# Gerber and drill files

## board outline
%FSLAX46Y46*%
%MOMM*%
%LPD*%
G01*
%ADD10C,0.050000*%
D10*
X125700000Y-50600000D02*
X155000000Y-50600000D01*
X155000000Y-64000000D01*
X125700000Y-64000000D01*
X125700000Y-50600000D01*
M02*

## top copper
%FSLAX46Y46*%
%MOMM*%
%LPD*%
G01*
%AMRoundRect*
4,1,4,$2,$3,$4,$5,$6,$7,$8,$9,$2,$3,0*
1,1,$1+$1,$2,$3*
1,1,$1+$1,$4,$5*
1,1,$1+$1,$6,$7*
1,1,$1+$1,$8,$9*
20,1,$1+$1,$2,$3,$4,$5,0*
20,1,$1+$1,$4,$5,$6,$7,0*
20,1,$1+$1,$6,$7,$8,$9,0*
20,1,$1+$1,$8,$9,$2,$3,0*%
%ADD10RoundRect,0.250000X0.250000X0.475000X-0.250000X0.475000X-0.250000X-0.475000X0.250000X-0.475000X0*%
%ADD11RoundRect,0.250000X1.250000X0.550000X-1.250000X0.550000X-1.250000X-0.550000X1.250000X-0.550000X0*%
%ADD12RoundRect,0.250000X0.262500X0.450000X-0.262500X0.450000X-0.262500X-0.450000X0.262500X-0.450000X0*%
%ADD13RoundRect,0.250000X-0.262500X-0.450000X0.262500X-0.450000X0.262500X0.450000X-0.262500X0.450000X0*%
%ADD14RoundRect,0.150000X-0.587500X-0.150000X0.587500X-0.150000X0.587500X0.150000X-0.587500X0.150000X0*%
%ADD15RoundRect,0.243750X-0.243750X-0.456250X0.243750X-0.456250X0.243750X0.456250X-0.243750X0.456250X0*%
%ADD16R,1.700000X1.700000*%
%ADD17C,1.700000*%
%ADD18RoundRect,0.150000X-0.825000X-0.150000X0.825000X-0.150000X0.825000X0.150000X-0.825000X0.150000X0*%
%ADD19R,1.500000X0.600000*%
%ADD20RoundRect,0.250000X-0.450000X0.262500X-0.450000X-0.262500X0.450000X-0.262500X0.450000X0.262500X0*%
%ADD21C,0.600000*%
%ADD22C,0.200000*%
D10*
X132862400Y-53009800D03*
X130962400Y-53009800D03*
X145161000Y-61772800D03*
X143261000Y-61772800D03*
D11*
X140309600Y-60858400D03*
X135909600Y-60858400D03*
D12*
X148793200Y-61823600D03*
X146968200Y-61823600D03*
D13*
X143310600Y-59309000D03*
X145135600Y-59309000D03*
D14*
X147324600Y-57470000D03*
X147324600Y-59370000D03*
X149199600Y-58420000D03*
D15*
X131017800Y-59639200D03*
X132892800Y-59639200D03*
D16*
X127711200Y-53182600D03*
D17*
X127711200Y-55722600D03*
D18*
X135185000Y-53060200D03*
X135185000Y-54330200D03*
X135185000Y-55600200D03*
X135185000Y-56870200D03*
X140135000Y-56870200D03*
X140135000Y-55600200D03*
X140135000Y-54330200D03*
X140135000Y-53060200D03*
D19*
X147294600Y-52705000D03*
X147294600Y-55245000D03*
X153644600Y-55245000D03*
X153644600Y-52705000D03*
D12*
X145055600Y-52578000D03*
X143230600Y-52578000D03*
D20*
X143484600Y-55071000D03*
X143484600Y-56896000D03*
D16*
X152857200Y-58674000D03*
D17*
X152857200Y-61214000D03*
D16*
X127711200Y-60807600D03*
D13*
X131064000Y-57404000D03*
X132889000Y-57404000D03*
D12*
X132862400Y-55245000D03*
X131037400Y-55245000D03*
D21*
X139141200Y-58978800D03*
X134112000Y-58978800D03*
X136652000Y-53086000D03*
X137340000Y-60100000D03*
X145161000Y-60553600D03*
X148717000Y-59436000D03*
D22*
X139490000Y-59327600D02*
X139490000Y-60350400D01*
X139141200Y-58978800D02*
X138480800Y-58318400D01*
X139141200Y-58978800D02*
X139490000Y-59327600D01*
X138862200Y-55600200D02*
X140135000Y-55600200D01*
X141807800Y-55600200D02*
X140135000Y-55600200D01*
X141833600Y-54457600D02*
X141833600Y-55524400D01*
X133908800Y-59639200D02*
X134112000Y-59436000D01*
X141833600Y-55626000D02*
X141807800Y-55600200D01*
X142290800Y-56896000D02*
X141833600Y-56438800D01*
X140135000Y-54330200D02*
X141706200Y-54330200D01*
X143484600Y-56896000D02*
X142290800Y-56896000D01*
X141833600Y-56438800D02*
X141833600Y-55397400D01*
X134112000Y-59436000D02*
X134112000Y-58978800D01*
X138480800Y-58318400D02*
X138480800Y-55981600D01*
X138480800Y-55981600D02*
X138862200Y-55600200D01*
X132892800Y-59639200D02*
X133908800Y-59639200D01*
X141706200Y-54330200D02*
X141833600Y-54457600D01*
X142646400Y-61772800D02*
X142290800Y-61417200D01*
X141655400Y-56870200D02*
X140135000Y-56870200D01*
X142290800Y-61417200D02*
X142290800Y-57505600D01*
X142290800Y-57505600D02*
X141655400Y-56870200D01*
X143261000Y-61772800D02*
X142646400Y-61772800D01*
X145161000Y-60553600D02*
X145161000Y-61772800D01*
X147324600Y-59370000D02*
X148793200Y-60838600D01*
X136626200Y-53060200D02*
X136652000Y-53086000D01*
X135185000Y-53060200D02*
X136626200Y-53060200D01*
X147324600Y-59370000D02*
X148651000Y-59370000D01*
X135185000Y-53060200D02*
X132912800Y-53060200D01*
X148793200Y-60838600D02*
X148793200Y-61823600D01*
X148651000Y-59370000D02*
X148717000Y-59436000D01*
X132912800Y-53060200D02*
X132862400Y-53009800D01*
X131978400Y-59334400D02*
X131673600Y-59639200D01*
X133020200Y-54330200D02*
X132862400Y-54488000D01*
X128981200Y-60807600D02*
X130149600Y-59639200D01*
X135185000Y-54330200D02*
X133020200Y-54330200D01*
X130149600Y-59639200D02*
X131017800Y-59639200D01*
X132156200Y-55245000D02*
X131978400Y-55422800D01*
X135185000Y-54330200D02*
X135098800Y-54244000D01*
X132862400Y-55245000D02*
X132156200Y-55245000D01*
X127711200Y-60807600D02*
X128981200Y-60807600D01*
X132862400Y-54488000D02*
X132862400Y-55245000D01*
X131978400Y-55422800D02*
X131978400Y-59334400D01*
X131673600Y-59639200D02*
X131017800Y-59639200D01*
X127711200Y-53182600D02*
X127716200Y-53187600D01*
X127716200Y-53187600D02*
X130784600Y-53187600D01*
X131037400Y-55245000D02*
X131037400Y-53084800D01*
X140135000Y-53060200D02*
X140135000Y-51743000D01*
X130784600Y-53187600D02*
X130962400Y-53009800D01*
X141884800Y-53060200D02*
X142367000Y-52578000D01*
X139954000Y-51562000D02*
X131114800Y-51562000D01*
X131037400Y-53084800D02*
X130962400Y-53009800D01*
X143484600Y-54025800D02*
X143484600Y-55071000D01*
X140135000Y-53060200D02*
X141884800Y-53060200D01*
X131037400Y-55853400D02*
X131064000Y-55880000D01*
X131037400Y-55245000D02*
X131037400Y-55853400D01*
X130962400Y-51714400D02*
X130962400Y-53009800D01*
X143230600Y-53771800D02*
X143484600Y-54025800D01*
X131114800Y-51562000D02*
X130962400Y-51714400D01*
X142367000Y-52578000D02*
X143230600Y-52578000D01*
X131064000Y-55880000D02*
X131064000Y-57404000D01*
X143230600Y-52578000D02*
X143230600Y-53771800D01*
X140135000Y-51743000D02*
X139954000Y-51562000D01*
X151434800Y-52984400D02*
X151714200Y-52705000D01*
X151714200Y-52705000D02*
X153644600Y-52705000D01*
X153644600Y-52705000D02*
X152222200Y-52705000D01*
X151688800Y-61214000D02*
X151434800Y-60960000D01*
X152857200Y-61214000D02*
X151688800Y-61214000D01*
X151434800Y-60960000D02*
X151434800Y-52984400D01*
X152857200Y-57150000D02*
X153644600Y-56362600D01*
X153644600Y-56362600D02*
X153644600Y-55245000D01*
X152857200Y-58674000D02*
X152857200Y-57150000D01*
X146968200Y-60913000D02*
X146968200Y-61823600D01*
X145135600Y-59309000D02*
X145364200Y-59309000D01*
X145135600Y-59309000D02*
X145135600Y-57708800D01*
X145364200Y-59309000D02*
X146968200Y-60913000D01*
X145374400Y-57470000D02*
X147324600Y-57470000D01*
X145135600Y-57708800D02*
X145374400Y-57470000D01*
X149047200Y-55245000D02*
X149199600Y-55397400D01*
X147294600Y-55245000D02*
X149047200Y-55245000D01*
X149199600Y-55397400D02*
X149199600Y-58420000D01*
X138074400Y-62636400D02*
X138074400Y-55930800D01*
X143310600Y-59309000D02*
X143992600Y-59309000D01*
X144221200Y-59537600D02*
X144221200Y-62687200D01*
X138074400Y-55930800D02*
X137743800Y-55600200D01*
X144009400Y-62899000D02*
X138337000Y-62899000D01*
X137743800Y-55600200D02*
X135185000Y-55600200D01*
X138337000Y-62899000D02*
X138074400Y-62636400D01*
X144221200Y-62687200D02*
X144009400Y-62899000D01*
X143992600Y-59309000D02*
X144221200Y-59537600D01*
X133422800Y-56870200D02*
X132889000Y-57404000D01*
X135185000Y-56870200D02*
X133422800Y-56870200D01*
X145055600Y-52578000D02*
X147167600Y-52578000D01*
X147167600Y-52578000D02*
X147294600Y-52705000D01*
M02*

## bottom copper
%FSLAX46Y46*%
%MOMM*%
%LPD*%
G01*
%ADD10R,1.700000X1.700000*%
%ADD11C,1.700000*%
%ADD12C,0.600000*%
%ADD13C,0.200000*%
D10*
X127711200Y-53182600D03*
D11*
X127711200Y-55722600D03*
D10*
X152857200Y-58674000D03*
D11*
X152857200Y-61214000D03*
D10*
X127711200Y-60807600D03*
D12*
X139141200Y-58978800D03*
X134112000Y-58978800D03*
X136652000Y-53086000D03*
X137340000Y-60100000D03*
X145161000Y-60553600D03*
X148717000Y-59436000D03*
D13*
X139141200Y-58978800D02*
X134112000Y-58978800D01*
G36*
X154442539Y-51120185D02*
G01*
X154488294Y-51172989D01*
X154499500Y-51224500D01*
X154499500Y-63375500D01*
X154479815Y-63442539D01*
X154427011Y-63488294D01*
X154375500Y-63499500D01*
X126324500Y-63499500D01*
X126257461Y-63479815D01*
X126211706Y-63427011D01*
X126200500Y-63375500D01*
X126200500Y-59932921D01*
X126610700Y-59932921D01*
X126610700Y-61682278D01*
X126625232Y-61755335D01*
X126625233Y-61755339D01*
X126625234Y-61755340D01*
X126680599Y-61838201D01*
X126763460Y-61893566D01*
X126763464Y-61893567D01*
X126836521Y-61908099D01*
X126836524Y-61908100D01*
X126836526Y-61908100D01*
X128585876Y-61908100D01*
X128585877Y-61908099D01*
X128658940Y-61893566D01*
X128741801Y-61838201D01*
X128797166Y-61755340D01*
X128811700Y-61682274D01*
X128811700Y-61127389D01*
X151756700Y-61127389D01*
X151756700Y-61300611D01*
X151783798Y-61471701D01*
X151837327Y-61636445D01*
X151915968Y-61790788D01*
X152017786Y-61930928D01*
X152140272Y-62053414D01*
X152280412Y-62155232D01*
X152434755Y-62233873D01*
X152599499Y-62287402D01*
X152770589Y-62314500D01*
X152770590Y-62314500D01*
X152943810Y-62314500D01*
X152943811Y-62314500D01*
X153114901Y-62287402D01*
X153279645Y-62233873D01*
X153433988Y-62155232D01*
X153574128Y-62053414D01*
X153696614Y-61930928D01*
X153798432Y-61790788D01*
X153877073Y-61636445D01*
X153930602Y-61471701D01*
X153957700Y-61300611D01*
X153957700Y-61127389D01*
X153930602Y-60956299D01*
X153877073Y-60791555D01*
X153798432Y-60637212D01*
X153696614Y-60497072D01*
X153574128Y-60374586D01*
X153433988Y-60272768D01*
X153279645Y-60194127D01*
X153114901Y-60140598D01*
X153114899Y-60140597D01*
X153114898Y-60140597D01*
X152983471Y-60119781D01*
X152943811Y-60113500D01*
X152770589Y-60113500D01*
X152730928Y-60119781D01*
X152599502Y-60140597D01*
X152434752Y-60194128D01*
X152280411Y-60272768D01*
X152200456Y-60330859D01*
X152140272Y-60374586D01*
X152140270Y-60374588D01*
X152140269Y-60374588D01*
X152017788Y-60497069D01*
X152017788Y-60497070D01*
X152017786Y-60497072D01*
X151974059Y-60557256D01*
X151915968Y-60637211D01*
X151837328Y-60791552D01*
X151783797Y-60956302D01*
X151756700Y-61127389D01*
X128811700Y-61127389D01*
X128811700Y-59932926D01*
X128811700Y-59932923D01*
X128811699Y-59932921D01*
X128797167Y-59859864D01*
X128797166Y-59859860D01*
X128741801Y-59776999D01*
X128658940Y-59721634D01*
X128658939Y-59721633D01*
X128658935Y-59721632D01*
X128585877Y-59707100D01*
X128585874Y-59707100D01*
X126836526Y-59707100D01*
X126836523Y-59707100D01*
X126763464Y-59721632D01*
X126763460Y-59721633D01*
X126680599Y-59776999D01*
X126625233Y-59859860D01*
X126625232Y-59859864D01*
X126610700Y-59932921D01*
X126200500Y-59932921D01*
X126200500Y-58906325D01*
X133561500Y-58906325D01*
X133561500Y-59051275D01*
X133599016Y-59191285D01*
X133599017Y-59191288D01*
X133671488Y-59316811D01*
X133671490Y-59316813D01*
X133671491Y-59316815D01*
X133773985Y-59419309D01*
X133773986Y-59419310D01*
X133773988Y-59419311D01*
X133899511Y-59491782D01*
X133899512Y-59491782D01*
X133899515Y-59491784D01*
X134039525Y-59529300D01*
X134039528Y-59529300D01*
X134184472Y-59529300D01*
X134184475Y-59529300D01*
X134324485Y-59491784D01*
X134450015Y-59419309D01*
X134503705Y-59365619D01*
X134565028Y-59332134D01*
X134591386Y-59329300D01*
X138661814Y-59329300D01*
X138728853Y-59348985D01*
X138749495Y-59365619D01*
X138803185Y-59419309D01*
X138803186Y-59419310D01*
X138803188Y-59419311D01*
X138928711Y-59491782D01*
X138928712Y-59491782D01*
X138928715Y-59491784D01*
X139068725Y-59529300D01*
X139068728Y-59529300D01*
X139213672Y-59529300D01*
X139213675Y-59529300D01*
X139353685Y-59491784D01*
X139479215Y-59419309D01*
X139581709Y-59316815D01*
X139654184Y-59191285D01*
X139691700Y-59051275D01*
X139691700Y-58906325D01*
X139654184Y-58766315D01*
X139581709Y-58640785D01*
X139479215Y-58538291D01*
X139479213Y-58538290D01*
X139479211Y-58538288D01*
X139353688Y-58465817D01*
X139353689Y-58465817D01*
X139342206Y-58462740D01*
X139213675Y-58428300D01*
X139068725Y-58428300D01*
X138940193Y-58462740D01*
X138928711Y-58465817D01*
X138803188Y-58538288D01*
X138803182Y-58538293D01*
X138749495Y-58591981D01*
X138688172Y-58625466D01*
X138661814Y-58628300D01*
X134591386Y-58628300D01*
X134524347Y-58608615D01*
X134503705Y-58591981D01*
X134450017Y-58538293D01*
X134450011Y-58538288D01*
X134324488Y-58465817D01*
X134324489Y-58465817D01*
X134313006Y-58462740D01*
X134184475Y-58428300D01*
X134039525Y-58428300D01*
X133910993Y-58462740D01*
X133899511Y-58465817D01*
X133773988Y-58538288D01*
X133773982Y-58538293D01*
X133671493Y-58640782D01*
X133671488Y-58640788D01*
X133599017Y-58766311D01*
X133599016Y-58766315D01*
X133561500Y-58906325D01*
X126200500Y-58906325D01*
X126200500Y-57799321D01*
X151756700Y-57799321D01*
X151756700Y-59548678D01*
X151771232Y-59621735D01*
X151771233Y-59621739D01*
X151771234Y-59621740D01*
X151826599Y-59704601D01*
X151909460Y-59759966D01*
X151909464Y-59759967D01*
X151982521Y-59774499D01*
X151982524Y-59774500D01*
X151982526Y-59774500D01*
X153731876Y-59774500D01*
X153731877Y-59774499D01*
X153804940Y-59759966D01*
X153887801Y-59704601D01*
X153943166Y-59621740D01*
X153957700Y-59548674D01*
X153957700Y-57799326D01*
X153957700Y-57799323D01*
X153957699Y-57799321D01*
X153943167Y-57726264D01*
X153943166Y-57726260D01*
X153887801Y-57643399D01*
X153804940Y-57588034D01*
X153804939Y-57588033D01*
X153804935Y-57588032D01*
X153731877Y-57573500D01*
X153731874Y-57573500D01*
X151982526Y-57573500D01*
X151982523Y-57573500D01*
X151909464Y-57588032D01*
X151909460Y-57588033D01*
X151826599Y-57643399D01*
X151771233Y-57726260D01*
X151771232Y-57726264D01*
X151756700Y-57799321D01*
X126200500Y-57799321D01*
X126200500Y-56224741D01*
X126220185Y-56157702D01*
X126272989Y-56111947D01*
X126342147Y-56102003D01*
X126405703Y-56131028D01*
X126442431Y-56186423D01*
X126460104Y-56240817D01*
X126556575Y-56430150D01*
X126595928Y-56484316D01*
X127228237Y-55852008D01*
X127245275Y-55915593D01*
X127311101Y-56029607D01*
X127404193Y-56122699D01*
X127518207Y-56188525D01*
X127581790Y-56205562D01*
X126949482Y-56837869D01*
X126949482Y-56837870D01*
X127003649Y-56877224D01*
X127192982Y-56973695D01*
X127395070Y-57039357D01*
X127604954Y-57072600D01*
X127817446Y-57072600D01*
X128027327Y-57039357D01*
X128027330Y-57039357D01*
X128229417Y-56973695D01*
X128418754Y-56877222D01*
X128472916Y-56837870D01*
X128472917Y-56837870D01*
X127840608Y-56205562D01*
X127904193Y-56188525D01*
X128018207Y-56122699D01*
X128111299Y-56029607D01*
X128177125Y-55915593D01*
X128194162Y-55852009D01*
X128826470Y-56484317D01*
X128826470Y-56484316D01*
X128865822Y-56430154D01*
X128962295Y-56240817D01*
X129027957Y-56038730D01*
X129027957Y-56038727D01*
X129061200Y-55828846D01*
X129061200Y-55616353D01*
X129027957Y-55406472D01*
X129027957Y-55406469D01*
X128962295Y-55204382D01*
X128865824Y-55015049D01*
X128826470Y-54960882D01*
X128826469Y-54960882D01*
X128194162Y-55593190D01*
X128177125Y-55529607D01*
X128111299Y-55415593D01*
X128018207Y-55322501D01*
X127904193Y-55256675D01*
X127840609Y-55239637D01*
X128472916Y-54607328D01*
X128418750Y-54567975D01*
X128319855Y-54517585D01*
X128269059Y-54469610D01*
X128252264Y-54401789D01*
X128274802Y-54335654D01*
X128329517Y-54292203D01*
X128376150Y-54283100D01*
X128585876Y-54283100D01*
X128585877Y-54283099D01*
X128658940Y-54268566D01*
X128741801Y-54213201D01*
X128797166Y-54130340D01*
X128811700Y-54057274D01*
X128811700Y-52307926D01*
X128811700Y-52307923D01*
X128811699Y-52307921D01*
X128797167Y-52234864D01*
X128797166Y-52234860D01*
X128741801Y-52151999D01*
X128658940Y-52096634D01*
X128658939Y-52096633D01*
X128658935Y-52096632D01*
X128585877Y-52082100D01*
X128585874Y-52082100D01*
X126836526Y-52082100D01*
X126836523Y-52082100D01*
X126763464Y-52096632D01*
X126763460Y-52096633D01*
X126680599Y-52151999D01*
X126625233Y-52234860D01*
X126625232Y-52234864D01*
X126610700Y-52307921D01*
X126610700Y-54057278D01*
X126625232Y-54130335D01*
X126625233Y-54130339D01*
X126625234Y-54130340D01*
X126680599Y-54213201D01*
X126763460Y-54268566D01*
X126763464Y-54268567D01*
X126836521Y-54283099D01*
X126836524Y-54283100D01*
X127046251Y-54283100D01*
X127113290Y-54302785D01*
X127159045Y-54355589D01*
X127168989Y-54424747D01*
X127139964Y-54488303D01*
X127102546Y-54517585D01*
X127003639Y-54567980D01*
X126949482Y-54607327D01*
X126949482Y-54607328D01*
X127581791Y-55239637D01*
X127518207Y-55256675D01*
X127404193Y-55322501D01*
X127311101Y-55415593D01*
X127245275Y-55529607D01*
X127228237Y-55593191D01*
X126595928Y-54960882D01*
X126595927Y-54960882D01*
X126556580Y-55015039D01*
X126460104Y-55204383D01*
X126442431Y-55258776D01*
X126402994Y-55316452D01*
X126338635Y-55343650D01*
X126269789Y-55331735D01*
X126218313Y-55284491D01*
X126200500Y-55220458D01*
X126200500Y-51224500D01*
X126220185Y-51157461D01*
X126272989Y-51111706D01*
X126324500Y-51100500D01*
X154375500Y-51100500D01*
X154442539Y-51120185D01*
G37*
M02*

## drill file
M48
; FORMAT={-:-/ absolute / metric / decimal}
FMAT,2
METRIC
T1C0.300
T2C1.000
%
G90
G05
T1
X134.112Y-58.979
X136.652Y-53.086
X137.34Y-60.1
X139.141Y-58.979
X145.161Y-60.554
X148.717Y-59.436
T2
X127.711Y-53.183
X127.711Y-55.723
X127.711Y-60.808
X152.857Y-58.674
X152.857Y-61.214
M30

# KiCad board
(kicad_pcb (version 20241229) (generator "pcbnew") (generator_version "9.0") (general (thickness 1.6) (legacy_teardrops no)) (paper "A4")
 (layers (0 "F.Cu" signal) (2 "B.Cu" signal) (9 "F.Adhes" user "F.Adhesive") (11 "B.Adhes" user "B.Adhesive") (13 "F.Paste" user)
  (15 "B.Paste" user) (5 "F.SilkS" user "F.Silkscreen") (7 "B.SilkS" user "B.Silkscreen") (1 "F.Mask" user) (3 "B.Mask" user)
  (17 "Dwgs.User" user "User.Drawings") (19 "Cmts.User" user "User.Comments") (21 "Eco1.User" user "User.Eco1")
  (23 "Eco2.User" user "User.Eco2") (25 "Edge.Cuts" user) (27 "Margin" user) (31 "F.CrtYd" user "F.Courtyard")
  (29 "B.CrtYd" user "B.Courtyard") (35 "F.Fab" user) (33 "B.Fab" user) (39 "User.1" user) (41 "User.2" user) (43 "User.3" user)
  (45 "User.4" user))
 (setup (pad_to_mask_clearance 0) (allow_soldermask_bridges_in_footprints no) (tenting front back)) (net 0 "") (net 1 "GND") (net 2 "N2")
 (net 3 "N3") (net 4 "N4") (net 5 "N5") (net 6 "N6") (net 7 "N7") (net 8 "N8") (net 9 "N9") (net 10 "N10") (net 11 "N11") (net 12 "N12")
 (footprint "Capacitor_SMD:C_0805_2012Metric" (layer "F.Cu") (at 131.9124 53.0098 180)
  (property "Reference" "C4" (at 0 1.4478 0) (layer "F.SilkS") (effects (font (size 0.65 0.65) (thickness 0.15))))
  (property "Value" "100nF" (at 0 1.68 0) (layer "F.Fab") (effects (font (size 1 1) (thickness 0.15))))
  (pad "1" smd roundrect (at -0.95 0 180) (size 1 1.45) (layers "F.Cu" "F.Mask" "F.Paste") (roundrect_rratio 0.25) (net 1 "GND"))
  (pad "2" smd roundrect (at 0.95 0 180) (size 1 1.45) (layers "F.Cu" "F.Mask" "F.Paste") (roundrect_rratio 0.25) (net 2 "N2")))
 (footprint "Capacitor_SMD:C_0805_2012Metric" (layer "F.Cu") (at 144.211 61.7728 180)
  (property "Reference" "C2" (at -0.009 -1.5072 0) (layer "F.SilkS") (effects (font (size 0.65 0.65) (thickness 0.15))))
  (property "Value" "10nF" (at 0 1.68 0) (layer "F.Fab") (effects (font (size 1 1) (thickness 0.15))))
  (pad "1" smd roundrect (at -0.95 0 180) (size 1 1.45) (layers "F.Cu" "F.Mask" "F.Paste") (roundrect_rratio 0.25) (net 1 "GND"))
  (pad "2" smd roundrect (at 0.95 0 180) (size 1 1.45) (layers "F.Cu" "F.Mask" "F.Paste") (roundrect_rratio 0.25) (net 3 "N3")))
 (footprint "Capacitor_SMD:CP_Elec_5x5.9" (layer "F.Cu") (at 138.1096 60.8584 180)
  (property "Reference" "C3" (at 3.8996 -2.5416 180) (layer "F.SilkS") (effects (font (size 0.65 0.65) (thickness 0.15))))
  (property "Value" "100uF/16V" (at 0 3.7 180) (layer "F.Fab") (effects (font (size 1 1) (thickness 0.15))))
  (pad "1" smd roundrect (at -2.2 0 180) (size 3 1.6) (layers "F.Cu" "F.Mask" "F.Paste") (roundrect_rratio 0.15625) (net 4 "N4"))
  (pad "2" smd roundrect (at 2.2 0 180) (size 3 1.6) (layers "F.Cu" "F.Mask" "F.Paste") (roundrect_rratio 0.15625) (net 1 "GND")))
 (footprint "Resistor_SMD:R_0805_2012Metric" (layer "F.Cu") (at 147.8807 61.8236 180)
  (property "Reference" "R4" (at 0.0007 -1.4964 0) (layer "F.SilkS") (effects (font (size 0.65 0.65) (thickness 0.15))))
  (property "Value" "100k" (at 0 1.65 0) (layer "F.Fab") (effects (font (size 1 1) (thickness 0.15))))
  (pad "1" smd roundrect (at -0.9125 0 180) (size 1.025 1.4) (layers "F.Cu" "F.Mask" "F.Paste") (roundrect_rratio 0.243902) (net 1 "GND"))
  (pad "2" smd roundrect (at 0.9125 0 180) (size 1.025 1.4) (layers "F.Cu" "F.Mask" "F.Paste") (roundrect_rratio 0.243902) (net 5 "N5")))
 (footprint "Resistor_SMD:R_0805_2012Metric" (layer "F.Cu") (at 144.2231 59.309)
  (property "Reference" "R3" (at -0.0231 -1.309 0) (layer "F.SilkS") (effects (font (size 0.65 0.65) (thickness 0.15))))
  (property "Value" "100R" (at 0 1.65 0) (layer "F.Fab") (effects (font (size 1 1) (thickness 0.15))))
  (pad "1" smd roundrect (at -0.9125 0) (size 1.025 1.4) (layers "F.Cu" "F.Mask" "F.Paste") (roundrect_rratio 0.243902) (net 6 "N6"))
  (pad "2" smd roundrect (at 0.9125 0) (size 1.025 1.4) (layers "F.Cu" "F.Mask" "F.Paste") (roundrect_rratio 0.243902) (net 5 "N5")))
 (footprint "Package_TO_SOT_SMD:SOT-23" (layer "F.Cu") (at 148.2621 58.42)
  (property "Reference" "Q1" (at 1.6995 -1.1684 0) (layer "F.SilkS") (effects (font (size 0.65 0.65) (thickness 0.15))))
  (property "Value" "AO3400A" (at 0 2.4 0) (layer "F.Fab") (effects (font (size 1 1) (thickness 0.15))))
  (pad "1" smd roundrect (at -0.9375 -0.95) (size 1.475 0.6) (layers "F.Cu" "F.Mask" "F.Paste") (roundrect_rratio 0.25) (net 5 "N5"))
  (pad "2" smd roundrect (at -0.9375 0.95) (size 1.475 0.6) (layers "F.Cu" "F.Mask" "F.Paste") (roundrect_rratio 0.25) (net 1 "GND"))
  (pad "3" smd roundrect (at 0.9375 0) (size 1.475 0.6) (layers "F.Cu" "F.Mask" "F.Paste") (roundrect_rratio 0.25) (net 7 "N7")))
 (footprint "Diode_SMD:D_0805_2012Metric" (layer "F.Cu") (at 131.9553 59.6392)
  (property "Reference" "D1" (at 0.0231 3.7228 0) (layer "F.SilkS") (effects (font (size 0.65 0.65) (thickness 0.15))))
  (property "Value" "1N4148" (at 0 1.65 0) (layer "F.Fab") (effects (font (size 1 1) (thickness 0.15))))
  (pad "1" smd roundrect (at -0.9375 0) (size 0.975 1.4) (layers "F.Cu" "F.Mask" "F.Paste") (roundrect_rratio 0.25) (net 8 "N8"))
  (pad "2" smd roundrect (at 0.9375 0) (size 0.975 1.4) (layers "F.Cu" "F.Mask" "F.Paste") (roundrect_rratio 0.25) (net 4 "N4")))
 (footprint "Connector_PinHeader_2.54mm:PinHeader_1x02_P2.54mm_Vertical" (layer "F.Cu") (at 127.7112 53.1826)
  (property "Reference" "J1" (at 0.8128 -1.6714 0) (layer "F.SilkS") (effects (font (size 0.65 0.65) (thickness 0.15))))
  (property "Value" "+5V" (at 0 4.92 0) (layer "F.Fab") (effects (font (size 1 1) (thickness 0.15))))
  (pad "1" thru_hole rect (at 0 0) (size 1.7 1.7) (drill 1) (layers "*.Cu" "*.Mask") (remove_unused_layers no) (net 2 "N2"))
  (pad "2" thru_hole circle (at 0 2.54) (size 1.7 1.7) (drill 1) (layers "*.Cu" "*.Mask") (remove_unused_layers no) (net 1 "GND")))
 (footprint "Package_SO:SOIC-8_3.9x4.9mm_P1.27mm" (layer "F.Cu") (at 137.66 54.9652)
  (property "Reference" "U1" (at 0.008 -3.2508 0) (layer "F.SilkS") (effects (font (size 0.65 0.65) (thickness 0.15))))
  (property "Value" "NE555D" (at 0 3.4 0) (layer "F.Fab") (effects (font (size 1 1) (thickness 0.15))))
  (pad "1" smd roundrect (at -2.475 -1.905) (size 1.95 0.6) (layers "F.Cu" "F.Mask" "F.Paste") (roundrect_rratio 0.25) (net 1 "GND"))
  (pad "2" smd roundrect (at -2.475 -0.635) (size 1.95 0.6) (layers "F.Cu" "F.Mask" "F.Paste") (roundrect_rratio 0.25) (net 8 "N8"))
  (pad "3" smd roundrect (at -2.475 0.635) (size 1.95 0.6) (layers "F.Cu" "F.Mask" "F.Paste") (roundrect_rratio 0.25) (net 6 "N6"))
  (pad "4" smd roundrect (at -2.475 1.905) (size 1.95 0.6) (layers "F.Cu" "F.Mask" "F.Paste") (roundrect_rratio 0.25) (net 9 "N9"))
  (pad "5" smd roundrect (at 2.475 1.905) (size 1.95 0.6) (layers "F.Cu" "F.Mask" "F.Paste") (roundrect_rratio 0.25) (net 3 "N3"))
  (pad "6" smd roundrect (at 2.475 0.635) (size 1.95 0.6) (layers "F.Cu" "F.Mask" "F.Paste") (roundrect_rratio 0.25) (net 4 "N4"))
  (pad "7" smd roundrect (at 2.475 -0.635) (size 1.95 0.6) (layers "F.Cu" "F.Mask" "F.Paste") (roundrect_rratio 0.25) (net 4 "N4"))
  (pad "8" smd roundrect (at 2.475 -1.905) (size 1.95 0.6) (layers "F.Cu" "F.Mask" "F.Paste") (roundrect_rratio 0.25) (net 2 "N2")))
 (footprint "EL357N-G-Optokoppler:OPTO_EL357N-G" (layer "F.Cu") (at 150.4696 53.975)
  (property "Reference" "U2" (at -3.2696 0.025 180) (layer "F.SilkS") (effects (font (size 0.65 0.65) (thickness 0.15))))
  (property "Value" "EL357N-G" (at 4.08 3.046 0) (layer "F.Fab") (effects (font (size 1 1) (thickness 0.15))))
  (pad "1" smd rect (at -3.175 -1.27) (size 1.5 0.6) (layers "F.Cu" "F.Mask" "F.Paste") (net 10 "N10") (solder_mask_margin 0.102))
  (pad "2" smd rect (at -3.175 1.27) (size 1.5 0.6) (layers "F.Cu" "F.Mask" "F.Paste") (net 7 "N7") (solder_mask_margin 0.102))
  (pad "3" smd rect (at 3.175 1.27) (size 1.5 0.6) (layers "F.Cu" "F.Mask" "F.Paste") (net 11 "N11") (solder_mask_margin 0.102))
  (pad "4" smd rect (at 3.175 -1.27) (size 1.5 0.6) (layers "F.Cu" "F.Mask" "F.Paste") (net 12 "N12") (solder_mask_margin 0.102)))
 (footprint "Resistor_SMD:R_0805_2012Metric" (layer "F.Cu") (at 144.1431 52.578 180)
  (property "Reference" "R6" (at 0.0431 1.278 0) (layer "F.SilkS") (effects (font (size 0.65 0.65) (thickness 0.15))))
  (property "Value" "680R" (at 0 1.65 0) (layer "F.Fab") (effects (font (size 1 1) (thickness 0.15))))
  (pad "1" smd roundrect (at -0.9125 0 180) (size 1.025 1.4) (layers "F.Cu" "F.Mask" "F.Paste") (roundrect_rratio 0.243902) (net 10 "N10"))
  (pad "2" smd roundrect (at 0.9125 0 180) (size 1.025 1.4) (layers "F.Cu" "F.Mask" "F.Paste") (roundrect_rratio 0.243902) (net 2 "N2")))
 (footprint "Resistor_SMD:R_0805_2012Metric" (layer "F.Cu") (at 143.4846 55.9835 -90)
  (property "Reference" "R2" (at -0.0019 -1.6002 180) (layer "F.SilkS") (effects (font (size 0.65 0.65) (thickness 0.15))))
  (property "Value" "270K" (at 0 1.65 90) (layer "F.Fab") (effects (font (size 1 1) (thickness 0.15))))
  (pad "1" smd roundrect (at -0.9125 0 270) (size 1.025 1.4) (layers "F.Cu" "F.Mask" "F.Paste") (roundrect_rratio 0.243902) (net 2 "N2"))
  (pad "2" smd roundrect (at 0.9125 0 270) (size 1.025 1.4) (layers "F.Cu" "F.Mask" "F.Paste") (roundrect_rratio 0.243902) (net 4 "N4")))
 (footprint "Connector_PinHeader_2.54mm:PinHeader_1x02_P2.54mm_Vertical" (layer "F.Cu") (at 152.8572 58.674)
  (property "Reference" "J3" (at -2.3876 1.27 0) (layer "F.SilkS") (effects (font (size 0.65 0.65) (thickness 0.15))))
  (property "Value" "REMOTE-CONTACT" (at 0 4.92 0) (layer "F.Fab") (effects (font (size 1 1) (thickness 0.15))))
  (pad "1" thru_hole rect (at 0 0) (size 1.7 1.7) (drill 1) (layers "*.Cu" "*.Mask") (remove_unused_layers no) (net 11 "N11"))
  (pad "2" thru_hole circle (at 0 2.54) (size 1.7 1.7) (drill 1) (layers "*.Cu" "*.Mask") (remove_unused_layers no) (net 12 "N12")))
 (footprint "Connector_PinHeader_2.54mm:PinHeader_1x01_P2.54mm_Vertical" (layer "F.Cu") (at 127.7112 60.8076)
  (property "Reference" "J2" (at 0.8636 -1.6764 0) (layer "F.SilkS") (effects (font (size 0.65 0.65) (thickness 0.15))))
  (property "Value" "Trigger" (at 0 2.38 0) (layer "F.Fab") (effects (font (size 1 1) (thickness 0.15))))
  (pad "1" thru_hole rect (at 0 0) (size 1.7 1.7) (drill 1) (layers "*.Cu" "*.Mask") (remove_unused_layers no) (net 8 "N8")))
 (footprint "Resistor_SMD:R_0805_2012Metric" (layer "F.Cu") (at 131.9765 57.404)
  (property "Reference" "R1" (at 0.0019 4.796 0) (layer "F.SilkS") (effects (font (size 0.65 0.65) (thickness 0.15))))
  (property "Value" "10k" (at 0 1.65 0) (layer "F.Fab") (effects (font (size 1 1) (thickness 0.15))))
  (pad "1" smd roundrect (at -0.9125 0) (size 1.025 1.4) (layers "F.Cu" "F.Mask" "F.Paste") (roundrect_rratio 0.243902) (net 2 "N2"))
  (pad "2" smd roundrect (at 0.9125 0) (size 1.025 1.4) (layers "F.Cu" "F.Mask" "F.Paste") (roundrect_rratio 0.243902) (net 9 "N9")))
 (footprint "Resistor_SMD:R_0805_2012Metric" (layer "F.Cu") (at 131.9499 55.245 180)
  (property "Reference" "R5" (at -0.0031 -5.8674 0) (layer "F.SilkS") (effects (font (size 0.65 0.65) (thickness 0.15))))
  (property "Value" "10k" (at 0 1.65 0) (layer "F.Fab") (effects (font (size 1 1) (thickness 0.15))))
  (pad "1" smd roundrect (at -0.9125 0 180) (size 1.025 1.4) (layers "F.Cu" "F.Mask" "F.Paste") (roundrect_rratio 0.243902) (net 8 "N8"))
  (pad "2" smd roundrect (at 0.9125 0 180) (size 1.025 1.4) (layers "F.Cu" "F.Mask" "F.Paste") (roundrect_rratio 0.243902) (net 2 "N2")))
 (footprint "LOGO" (layer "B.Cu") (at 140.84617 57.489081 180)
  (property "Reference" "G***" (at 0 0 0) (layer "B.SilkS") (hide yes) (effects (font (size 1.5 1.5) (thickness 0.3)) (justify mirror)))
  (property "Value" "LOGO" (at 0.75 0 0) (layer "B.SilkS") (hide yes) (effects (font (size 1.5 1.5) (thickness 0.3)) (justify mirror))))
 (gr_rect (start 125.7 50.6) (end 155 64) (stroke (width 0.05) (type default)) (fill no) (layer "Edge.Cuts"))
 (segment (start 139.49 59.3276) (end 139.49 60.3504) (width 0.2) (layer "F.Cu") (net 4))
 (segment (start 139.1412 58.9788) (end 138.4808 58.3184) (width 0.2) (layer "F.Cu") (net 4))
 (segment (start 139.1412 58.9788) (end 139.49 59.3276) (width 0.2) (layer "F.Cu") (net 4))
 (segment (start 138.8622 55.6002) (end 140.135 55.6002) (width 0.2) (layer "F.Cu") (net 4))
 (segment (start 141.8078 55.6002) (end 140.135 55.6002) (width 0.2) (layer "F.Cu") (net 4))
 (segment (start 141.8336 54.4576) (end 141.8336 55.5244) (width 0.2) (layer "F.Cu") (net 4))
 (segment (start 133.9088 59.6392) (end 134.112 59.436) (width 0.2) (layer "F.Cu") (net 4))
 (segment (start 141.8336 55.626) (end 141.8078 55.6002) (width 0.2) (layer "F.Cu") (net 4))
 (segment (start 142.2908 56.896) (end 141.8336 56.4388) (width 0.2) (layer "F.Cu") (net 4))
 (segment (start 140.135 54.3302) (end 141.7062 54.3302) (width 0.2) (layer "F.Cu") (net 4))
 (segment (start 143.4846 56.896) (end 142.2908 56.896) (width 0.2) (layer "F.Cu") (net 4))
 (segment (start 141.8336 56.4388) (end 141.8336 55.3974) (width 0.2) (layer "F.Cu") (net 4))
 (segment (start 134.112 59.436) (end 134.112 58.9788) (width 0.2) (layer "F.Cu") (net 4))
 (segment (start 138.4808 58.3184) (end 138.4808 55.9816) (width 0.2) (layer "F.Cu") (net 4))
 (segment (start 138.4808 55.9816) (end 138.8622 55.6002) (width 0.2) (layer "F.Cu") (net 4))
 (segment (start 132.8928 59.6392) (end 133.9088 59.6392) (width 0.2) (layer "F.Cu") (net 4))
 (segment (start 141.7062 54.3302) (end 141.8336 54.4576) (width 0.2) (layer "F.Cu") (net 4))
 (via (at 139.1412 58.9788) (size 0.6) (drill 0.3) (layers "F.Cu" "B.Cu") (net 4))
 (via (at 134.112 58.9788) (size 0.6) (drill 0.3) (layers "F.Cu" "B.Cu") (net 4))
 (segment (start 139.1412 58.9788) (end 134.112 58.9788) (width 0.2) (layer "B.Cu") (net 4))
 (segment (start 142.6464 61.7728) (end 142.2908 61.4172) (width 0.2) (layer "F.Cu") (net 3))
 (segment (start 141.6554 56.8702) (end 140.135 56.8702) (width 0.2) (layer "F.Cu") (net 3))
 (segment (start 142.2908 61.4172) (end 142.2908 57.5056) (width 0.2) (layer "F.Cu") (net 3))
 (segment (start 142.2908 57.5056) (end 141.6554 56.8702) (width 0.2) (layer "F.Cu") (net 3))
 (segment (start 143.261 61.7728) (end 142.6464 61.7728) (width 0.2) (layer "F.Cu") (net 3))
 (segment (start 145.161 60.5536) (end 145.161 61.7728) (width 0.2) (layer "F.Cu") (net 1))
 (segment (start 147.3246 59.37) (end 148.7932 60.8386) (width 0.2) (layer "F.Cu") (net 1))
 (segment (start 136.6262 53.0602) (end 136.652 53.086) (width 0.2) (layer "F.Cu") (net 1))
 (segment (start 135.185 53.0602) (end 136.6262 53.0602) (width 0.2) (layer "F.Cu") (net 1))
 (segment (start 147.3246 59.37) (end 148.651 59.37) (width 0.2) (layer "F.Cu") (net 1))
 (segment (start 135.185 53.0602) (end 132.9128 53.0602) (width 0.2) (layer "F.Cu") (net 1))
 (segment (start 148.7932 60.8386) (end 148.7932 61.8236) (width 0.2) (layer "F.Cu") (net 1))
 (segment (start 148.651 59.37) (end 148.717 59.436) (width 0.2) (layer "F.Cu") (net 1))
 (segment (start 132.9128 53.0602) (end 132.8624 53.0098) (width 0.2) (layer "F.Cu") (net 1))
 (via (at 136.652 53.086) (size 0.6) (drill 0.3) (layers "F.Cu" "B.Cu") (free yes) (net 1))
 (via (at 137.34 60.1) (size 0.6) (drill 0.3) (layers "F.Cu" "B.Cu") (free yes) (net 1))
 (via (at 145.161 60.5536) (size 0.6) (drill 0.3) (layers "F.Cu" "B.Cu") (free yes) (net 1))
 (via (at 148.717 59.436) (size 0.6) (drill 0.3) (layers "F.Cu" "B.Cu") (free yes) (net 1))
 (segment (start 131.9784 59.3344) (end 131.6736 59.6392) (width 0.2) (layer "F.Cu") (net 8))
 (segment (start 133.0202 54.3302) (end 132.8624 54.488) (width 0.2) (layer "F.Cu") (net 8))
 (segment (start 128.9812 60.8076) (end 130.1496 59.6392) (width 0.2) (layer "F.Cu") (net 8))
 (segment (start 135.185 54.3302) (end 133.0202 54.3302) (width 0.2) (layer "F.Cu") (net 8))
 (segment (start 130.1496 59.6392) (end 131.0178 59.6392) (width 0.2) (layer "F.Cu") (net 8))
 (segment (start 132.1562 55.245) (end 131.9784 55.4228) (width 0.2) (layer "F.Cu") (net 8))
 (segment (start 135.185 54.3302) (end 135.0988 54.244) (width 0.2) (layer "F.Cu") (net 8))
 (segment (start 132.8624 55.245) (end 132.1562 55.245) (width 0.2) (layer "F.Cu") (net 8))
 (segment (start 127.7112 60.8076) (end 128.9812 60.8076) (width 0.2) (layer "F.Cu") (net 8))
 (segment (start 132.8624 54.488) (end 132.8624 55.245) (width 0.2) (layer "F.Cu") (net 8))
 (segment (start 131.9784 55.4228) (end 131.9784 59.3344) (width 0.2) (layer "F.Cu") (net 8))
 (segment (start 131.6736 59.6392) (end 131.0178 59.6392) (width 0.2) (layer "F.Cu") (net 8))
 (segment (start 127.7112 53.1826) (end 127.7162 53.1876) (width 0.2) (layer "F.Cu") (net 2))
 (segment (start 127.7162 53.1876) (end 130.7846 53.1876) (width 0.2) (layer "F.Cu") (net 2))
 (segment (start 131.0374 55.245) (end 131.0374 53.0848) (width 0.2) (layer "F.Cu") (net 2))
 (segment (start 140.135 53.0602) (end 140.135 51.743) (width 0.2) (layer "F.Cu") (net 2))
 (segment (start 130.7846 53.1876) (end 130.9624 53.0098) (width 0.2) (layer "F.Cu") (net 2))
 (segment (start 141.8848 53.0602) (end 142.367 52.578) (width 0.2) (layer "F.Cu") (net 2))
 (segment (start 139.954 51.562) (end 131.1148 51.562) (width 0.2) (layer "F.Cu") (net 2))
 (segment (start 131.0374 53.0848) (end 130.9624 53.0098) (width 0.2) (layer "F.Cu") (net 2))
 (segment (start 143.4846 54.0258) (end 143.4846 55.071) (width 0.2) (layer "F.Cu") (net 2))
 (segment (start 140.135 53.0602) (end 141.8848 53.0602) (width 0.2) (layer "F.Cu") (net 2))
 (segment (start 131.0374 55.8534) (end 131.064 55.88) (width 0.2) (layer "F.Cu") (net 2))
 (segment (start 131.0374 55.245) (end 131.0374 55.8534) (width 0.2) (layer "F.Cu") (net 2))
 (segment (start 130.9624 51.7144) (end 130.9624 53.0098) (width 0.2) (layer "F.Cu") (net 2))
 (segment (start 143.2306 53.7718) (end 143.4846 54.0258) (width 0.2) (layer "F.Cu") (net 2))
 (segment (start 131.1148 51.562) (end 130.9624 51.7144) (width 0.2) (layer "F.Cu") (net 2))
 (segment (start 142.367 52.578) (end 143.2306 52.578) (width 0.2) (layer "F.Cu") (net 2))
 (segment (start 131.064 55.88) (end 131.064 57.404) (width 0.2) (layer "F.Cu") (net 2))
 (segment (start 143.2306 52.578) (end 143.2306 53.7718) (width 0.2) (layer "F.Cu") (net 2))
 (segment (start 140.135 51.743) (end 139.954 51.562) (width 0.2) (layer "F.Cu") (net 2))
 (segment (start 151.4348 52.9844) (end 151.7142 52.705) (width 0.2) (layer "F.Cu") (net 12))
 (segment (start 151.7142 52.705) (end 153.6446 52.705) (width 0.2) (layer "F.Cu") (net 12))
 (segment (start 153.6446 52.705) (end 152.2222 52.705) (width 0.2) (layer "F.Cu") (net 12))
 (segment (start 151.6888 61.214) (end 151.4348 60.96) (width 0.2) (layer "F.Cu") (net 12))
 (segment (start 152.8572 61.214) (end 151.6888 61.214) (width 0.2) (layer "F.Cu") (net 12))
 (segment (start 151.4348 60.96) (end 151.4348 52.9844) (width 0.2) (layer "F.Cu") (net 12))
 (segment (start 152.8572 57.15) (end 153.6446 56.3626) (width 0.2) (layer "F.Cu") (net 11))
 (segment (start 153.6446 56.3626) (end 153.6446 55.245) (width 0.2) (layer "F.Cu") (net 11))
 (segment (start 152.8572 58.674) (end 152.8572 57.15) (width 0.2) (layer "F.Cu") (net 11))
 (segment (start 146.9682 60.913) (end 146.9682 61.8236) (width 0.2) (layer "F.Cu") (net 5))
 (segment (start 145.1356 59.309) (end 145.3642 59.309) (width 0.2) (layer "F.Cu") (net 5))
 (segment (start 145.1356 59.309) (end 145.1356 57.7088) (width 0.2) (layer "F.Cu") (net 5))
 (segment (start 145.3642 59.309) (end 146.9682 60.913) (width 0.2) (layer "F.Cu") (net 5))
 (segment (start 145.3744 57.47) (end 147.3246 57.47) (width 0.2) (layer "F.Cu") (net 5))
 (segment (start 145.1356 57.7088) (end 145.3744 57.47) (width 0.2) (layer "F.Cu") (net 5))
 (segment (start 149.0472 55.245) (end 149.1996 55.3974) (width 0.2) (layer "F.Cu") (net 7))
 (segment (start 147.2946 55.245) (end 149.0472 55.245) (width 0.2) (layer "F.Cu") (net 7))
 (segment (start 149.1996 55.3974) (end 149.1996 58.42) (width 0.2) (layer "F.Cu") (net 7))
 (segment (start 138.0744 62.6364) (end 138.0744 55.9308) (width 0.2) (layer "F.Cu") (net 6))
 (segment (start 143.3106 59.309) (end 143.9926 59.309) (width 0.2) (layer "F.Cu") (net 6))
 (segment (start 144.2212 59.5376) (end 144.2212 62.6872) (width 0.2) (layer "F.Cu") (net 6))
 (segment (start 138.0744 55.9308) (end 137.7438 55.6002) (width 0.2) (layer "F.Cu") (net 6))
 (segment (start 144.0094 62.899) (end 138.337 62.899) (width 0.2) (layer "F.Cu") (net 6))
 (segment (start 137.7438 55.6002) (end 135.185 55.6002) (width 0.2) (layer "F.Cu") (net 6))
 (segment (start 138.337 62.899) (end 138.0744 62.6364) (width 0.2) (layer "F.Cu") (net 6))
 (segment (start 144.2212 62.6872) (end 144.0094 62.899) (width 0.2) (layer "F.Cu") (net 6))
 (segment (start 143.9926 59.309) (end 144.2212 59.5376) (width 0.2) (layer "F.Cu") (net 6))
 (segment (start 133.4228 56.8702) (end 132.889 57.404) (width 0.2) (layer "F.Cu") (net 9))
 (segment (start 135.185 56.8702) (end 133.4228 56.8702) (width 0.2) (layer "F.Cu") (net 9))
 (segment (start 145.0556 52.578) (end 147.1676 52.578) (width 0.2) (layer "F.Cu") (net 10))
 (segment (start 147.1676 52.578) (end 147.2946 52.705) (width 0.2) (layer "F.Cu") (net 10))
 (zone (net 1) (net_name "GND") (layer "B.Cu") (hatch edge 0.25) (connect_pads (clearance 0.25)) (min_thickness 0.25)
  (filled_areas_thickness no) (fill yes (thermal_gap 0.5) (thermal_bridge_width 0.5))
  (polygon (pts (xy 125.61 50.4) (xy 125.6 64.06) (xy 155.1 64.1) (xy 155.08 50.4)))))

